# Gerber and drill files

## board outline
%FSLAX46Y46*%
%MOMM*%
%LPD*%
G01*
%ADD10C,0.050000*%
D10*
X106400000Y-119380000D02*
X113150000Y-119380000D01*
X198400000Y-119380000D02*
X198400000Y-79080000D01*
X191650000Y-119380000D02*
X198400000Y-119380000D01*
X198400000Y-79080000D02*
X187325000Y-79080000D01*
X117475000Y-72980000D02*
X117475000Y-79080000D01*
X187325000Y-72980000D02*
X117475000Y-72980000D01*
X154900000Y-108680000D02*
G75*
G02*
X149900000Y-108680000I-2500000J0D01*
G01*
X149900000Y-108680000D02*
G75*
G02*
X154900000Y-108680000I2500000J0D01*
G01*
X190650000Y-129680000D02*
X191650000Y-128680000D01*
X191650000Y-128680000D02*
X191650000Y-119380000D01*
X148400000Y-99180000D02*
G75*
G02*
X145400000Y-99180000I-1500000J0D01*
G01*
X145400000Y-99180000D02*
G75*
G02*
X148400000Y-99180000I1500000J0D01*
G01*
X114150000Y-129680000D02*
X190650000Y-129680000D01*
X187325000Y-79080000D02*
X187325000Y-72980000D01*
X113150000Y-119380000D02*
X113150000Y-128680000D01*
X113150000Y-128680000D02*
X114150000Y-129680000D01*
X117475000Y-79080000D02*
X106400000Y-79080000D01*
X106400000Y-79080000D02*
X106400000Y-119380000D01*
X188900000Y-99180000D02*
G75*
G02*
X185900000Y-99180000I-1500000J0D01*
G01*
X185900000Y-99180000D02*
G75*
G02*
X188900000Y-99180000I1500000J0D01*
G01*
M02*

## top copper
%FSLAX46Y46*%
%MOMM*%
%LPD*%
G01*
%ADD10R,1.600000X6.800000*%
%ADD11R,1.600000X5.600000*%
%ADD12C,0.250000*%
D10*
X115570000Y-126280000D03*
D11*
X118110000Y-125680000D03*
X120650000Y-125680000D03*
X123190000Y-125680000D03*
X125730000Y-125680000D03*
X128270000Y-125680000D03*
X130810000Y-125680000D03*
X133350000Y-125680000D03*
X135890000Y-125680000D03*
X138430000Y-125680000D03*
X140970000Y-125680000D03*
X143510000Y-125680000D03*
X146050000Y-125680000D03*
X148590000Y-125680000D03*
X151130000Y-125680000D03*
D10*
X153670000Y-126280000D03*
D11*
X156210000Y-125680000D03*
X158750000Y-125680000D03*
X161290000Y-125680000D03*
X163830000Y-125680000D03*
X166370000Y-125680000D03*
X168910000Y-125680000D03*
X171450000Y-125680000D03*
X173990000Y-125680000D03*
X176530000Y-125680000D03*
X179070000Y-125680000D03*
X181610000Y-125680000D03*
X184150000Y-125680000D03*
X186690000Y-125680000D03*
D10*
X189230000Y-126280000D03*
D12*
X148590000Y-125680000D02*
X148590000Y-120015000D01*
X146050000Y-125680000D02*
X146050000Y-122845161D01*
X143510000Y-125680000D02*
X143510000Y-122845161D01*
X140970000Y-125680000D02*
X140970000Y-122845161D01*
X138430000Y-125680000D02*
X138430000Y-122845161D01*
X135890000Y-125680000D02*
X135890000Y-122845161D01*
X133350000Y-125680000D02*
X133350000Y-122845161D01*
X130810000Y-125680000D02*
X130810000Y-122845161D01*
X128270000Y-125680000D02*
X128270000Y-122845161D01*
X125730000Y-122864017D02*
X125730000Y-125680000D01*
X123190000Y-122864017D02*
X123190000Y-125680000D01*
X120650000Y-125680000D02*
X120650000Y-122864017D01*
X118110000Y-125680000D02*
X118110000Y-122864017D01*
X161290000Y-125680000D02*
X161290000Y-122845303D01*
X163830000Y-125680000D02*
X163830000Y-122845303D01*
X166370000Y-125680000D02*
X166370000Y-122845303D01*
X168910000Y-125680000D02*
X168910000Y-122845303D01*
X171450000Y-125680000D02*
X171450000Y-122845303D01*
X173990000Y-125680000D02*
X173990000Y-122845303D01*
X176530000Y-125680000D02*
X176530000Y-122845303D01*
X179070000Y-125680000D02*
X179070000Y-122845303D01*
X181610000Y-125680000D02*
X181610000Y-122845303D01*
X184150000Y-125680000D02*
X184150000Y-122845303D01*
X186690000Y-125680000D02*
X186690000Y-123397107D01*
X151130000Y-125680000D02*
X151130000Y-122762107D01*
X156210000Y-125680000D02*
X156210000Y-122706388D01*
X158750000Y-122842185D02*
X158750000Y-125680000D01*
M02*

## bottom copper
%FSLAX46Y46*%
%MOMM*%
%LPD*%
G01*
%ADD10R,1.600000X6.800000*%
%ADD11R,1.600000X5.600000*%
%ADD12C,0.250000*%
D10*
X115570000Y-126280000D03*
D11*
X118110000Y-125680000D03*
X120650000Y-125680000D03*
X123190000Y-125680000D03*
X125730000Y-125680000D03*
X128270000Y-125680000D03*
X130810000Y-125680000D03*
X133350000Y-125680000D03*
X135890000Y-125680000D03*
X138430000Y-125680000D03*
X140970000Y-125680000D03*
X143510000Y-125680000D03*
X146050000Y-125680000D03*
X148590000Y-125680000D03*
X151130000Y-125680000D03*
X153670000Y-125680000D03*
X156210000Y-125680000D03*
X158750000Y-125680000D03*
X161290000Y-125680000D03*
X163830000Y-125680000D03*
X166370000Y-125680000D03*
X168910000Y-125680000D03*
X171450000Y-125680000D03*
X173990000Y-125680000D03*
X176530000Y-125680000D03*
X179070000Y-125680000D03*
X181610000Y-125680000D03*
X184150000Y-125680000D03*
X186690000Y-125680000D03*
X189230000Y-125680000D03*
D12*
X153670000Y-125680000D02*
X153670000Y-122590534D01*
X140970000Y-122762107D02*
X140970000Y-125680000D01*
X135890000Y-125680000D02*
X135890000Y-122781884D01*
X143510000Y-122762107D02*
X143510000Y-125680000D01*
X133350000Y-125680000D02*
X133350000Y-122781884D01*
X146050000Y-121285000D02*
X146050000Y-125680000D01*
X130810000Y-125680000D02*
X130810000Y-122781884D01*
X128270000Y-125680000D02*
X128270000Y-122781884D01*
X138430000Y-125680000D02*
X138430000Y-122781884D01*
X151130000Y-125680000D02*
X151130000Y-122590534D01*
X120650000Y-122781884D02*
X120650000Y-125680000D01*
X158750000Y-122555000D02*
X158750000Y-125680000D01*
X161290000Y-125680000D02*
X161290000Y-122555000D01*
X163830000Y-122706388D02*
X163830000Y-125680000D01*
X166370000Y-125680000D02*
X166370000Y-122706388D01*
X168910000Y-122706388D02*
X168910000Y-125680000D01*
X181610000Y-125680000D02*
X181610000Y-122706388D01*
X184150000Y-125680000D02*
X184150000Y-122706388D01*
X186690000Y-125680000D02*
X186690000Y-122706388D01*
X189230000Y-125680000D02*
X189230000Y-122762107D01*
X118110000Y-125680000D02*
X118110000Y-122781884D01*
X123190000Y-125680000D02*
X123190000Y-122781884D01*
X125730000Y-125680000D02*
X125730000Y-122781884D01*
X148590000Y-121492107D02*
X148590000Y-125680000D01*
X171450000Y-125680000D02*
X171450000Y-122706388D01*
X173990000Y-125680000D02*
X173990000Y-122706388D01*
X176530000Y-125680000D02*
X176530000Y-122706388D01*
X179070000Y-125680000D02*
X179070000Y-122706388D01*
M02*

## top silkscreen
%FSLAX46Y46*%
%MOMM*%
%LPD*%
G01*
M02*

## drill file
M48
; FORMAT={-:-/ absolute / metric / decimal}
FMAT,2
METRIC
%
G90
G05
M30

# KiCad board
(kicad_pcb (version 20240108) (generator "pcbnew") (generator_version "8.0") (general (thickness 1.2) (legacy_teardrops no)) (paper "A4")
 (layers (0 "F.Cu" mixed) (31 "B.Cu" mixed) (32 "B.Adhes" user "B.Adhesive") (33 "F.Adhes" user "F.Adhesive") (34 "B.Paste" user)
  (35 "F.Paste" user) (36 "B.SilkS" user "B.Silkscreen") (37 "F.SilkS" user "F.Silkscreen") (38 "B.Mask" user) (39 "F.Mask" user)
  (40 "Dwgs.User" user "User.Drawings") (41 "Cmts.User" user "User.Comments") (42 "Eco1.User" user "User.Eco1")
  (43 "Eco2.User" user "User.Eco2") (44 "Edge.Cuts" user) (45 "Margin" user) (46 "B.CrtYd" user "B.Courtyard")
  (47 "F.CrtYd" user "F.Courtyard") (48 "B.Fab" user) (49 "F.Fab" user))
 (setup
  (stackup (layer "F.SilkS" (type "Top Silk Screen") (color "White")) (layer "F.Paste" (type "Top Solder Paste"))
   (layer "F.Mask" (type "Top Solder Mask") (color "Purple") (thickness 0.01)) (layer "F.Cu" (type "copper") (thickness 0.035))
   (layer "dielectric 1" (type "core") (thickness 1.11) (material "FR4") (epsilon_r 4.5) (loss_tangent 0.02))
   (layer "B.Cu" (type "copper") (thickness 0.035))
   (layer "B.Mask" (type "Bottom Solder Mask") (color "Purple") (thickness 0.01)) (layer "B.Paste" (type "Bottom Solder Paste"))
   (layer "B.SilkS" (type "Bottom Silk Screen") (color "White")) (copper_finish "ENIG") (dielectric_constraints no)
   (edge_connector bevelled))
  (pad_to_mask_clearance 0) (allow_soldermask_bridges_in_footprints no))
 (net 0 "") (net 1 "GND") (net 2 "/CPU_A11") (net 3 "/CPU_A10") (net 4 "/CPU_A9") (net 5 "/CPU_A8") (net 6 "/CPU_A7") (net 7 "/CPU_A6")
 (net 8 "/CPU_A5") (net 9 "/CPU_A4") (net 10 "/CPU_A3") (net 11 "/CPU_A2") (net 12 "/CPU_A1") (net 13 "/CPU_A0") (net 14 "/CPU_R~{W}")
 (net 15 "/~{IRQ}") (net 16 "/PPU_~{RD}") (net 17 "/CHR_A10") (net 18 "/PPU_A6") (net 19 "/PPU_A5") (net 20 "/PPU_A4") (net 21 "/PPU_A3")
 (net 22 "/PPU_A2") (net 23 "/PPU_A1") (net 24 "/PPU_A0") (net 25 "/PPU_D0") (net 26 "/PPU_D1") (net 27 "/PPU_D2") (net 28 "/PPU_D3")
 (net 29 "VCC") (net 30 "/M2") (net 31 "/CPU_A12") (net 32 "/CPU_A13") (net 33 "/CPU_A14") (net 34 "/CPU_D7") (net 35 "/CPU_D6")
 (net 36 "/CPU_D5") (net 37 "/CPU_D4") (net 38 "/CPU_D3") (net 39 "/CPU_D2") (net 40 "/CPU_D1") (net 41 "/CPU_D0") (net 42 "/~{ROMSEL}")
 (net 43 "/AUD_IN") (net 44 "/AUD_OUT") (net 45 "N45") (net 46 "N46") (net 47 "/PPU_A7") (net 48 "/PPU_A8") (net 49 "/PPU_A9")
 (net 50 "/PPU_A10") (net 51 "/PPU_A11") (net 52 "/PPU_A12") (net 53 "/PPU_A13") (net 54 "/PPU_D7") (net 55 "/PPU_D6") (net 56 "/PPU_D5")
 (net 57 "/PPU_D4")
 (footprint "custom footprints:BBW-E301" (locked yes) (layer "F.Cu") (at 152.4 119.38)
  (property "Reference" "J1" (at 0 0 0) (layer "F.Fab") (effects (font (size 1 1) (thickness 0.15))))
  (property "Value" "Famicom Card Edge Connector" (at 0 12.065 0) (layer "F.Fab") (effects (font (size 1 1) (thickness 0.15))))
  (pad "1" connect rect (at -36.83 6.9) (size 1.6 6.8) (layers "F.Cu") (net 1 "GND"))
  (pad "2" connect rect (at -34.29 6.3) (size 1.6 5.6) (layers "F.Cu") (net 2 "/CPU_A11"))
  (pad "3" connect rect (at -31.75 6.3) (size 1.6 5.6) (layers "F.Cu") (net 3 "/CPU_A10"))
  (pad "4" connect rect (at -29.21 6.3) (size 1.6 5.6) (layers "F.Cu") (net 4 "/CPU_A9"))
  (pad "5" connect rect (at -26.67 6.3) (size 1.6 5.6) (layers "F.Cu") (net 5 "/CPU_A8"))
  (pad "6" connect rect (at -24.13 6.3) (size 1.6 5.6) (layers "F.Cu") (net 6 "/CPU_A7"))
  (pad "7" connect rect (at -21.59 6.3) (size 1.6 5.6) (layers "F.Cu") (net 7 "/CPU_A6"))
  (pad "8" connect rect (at -19.05 6.3) (size 1.6 5.6) (layers "F.Cu") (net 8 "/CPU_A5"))
  (pad "9" connect rect (at -16.51 6.3) (size 1.6 5.6) (layers "F.Cu") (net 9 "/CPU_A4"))
  (pad "10" connect rect (at -13.97 6.3) (size 1.6 5.6) (layers "F.Cu") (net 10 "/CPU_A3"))
  (pad "11" connect rect (at -11.43 6.3) (size 1.6 5.6) (layers "F.Cu") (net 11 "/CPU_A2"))
  (pad "12" connect rect (at -8.89 6.3) (size 1.6 5.6) (layers "F.Cu") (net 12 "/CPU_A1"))
  (pad "13" connect rect (at -6.35 6.3) (size 1.6 5.6) (layers "F.Cu") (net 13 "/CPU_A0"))
  (pad "14" connect rect (at -3.81 6.3) (size 1.6 5.6) (layers "F.Cu") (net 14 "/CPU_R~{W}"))
  (pad "15" connect rect (at -1.27 6.3) (size 1.6 5.6) (layers "F.Cu") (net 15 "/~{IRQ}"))
  (pad "16" connect rect (at 1.27 6.9) (size 1.6 6.8) (layers "F.Cu") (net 1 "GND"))
  (pad "17" connect rect (at 3.81 6.3) (size 1.6 5.6) (layers "F.Cu") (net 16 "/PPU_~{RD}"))
  (pad "18" connect rect (at 6.35 6.3) (size 1.6 5.6) (layers "F.Cu") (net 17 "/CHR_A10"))
  (pad "19" connect rect (at 8.89 6.3) (size 1.6 5.6) (layers "F.Cu") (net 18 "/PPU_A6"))
  (pad "20" connect rect (at 11.43 6.3) (size 1.6 5.6) (layers "F.Cu") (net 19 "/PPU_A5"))
  (pad "21" connect rect (at 13.97 6.3) (size 1.6 5.6) (layers "F.Cu") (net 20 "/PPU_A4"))
  (pad "22" connect rect (at 16.51 6.3) (size 1.6 5.6) (layers "F.Cu") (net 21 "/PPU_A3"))
  (pad "23" connect rect (at 19.05 6.3) (size 1.6 5.6) (layers "F.Cu") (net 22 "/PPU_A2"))
  (pad "24" connect rect (at 21.59 6.3) (size 1.6 5.6) (layers "F.Cu") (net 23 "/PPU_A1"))
  (pad "25" connect rect (at 24.13 6.3) (size 1.6 5.6) (layers "F.Cu") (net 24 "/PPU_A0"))
  (pad "26" connect rect (at 26.67 6.3) (size 1.6 5.6) (layers "F.Cu") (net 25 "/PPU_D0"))
  (pad "27" connect rect (at 29.21 6.3) (size 1.6 5.6) (layers "F.Cu") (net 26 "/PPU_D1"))
  (pad "28" connect rect (at 31.75 6.3) (size 1.6 5.6) (layers "F.Cu") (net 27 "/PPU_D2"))
  (pad "29" connect rect (at 34.29 6.3) (size 1.6 5.6) (layers "F.Cu") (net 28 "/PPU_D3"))
  (pad "30" connect rect (at 36.83 6.9) (size 1.6 6.8) (layers "F.Cu") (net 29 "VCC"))
  (pad "31" connect rect (at -36.83 6.9) (size 1.6 6.8) (layers "B.Cu") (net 29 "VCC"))
  (pad "32" connect rect (at -34.29 6.3) (size 1.6 5.6) (layers "B.Cu") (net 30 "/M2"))
  (pad "33" connect rect (at -31.75 6.3) (size 1.6 5.6) (layers "B.Cu") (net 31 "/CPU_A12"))
  (pad "34" connect rect (at -29.21 6.3) (size 1.6 5.6) (layers "B.Cu") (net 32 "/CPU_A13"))
  (pad "35" connect rect (at -26.67 6.3) (size 1.6 5.6) (layers "B.Cu") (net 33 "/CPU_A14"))
  (pad "36" connect rect (at -24.13 6.3) (size 1.6 5.6) (layers "B.Cu") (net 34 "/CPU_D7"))
  (pad "37" connect rect (at -21.59 6.3) (size 1.6 5.6) (layers "B.Cu") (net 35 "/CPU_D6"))
  (pad "38" connect rect (at -19.05 6.3) (size 1.6 5.6) (layers "B.Cu") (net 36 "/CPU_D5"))
  (pad "39" connect rect (at -16.51 6.3) (size 1.6 5.6) (layers "B.Cu") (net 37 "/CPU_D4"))
  (pad "40" connect rect (at -13.97 6.3) (size 1.6 5.6) (layers "B.Cu") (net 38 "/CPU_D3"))
  (pad "41" connect rect (at -11.43 6.3) (size 1.6 5.6) (layers "B.Cu") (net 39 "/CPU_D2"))
  (pad "42" connect rect (at -8.89 6.3) (size 1.6 5.6) (layers "B.Cu") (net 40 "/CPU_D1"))
  (pad "43" connect rect (at -6.35 6.3) (size 1.6 5.6) (layers "B.Cu") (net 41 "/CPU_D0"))
  (pad "44" connect rect (at -3.81 6.3) (size 1.6 5.6) (layers "B.Cu") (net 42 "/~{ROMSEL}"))
  (pad "45" connect rect (at -1.27 6.3) (size 1.6 5.6) (layers "B.Cu") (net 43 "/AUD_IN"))
  (pad "46" connect rect (at 1.27 6.3) (size 1.6 5.6) (layers "B.Cu") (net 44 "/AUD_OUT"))
  (pad "47" connect rect (at 3.81 6.3) (size 1.6 5.6) (layers "B.Cu") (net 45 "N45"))
  (pad "48" connect rect (at 6.35 6.3) (size 1.6 5.6) (layers "B.Cu") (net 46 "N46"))
  (pad "49" connect rect (at 8.89 6.3) (size 1.6 5.6) (layers "B.Cu") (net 46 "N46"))
  (pad "50" connect rect (at 11.43 6.3) (size 1.6 5.6) (layers "B.Cu") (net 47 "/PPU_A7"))
  (pad "51" connect rect (at 13.97 6.3) (size 1.6 5.6) (layers "B.Cu") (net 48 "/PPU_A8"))
  (pad "52" connect rect (at 16.51 6.3) (size 1.6 5.6) (layers "B.Cu") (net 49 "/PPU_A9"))
  (pad "53" connect rect (at 19.05 6.3) (size 1.6 5.6) (layers "B.Cu") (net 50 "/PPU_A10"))
  (pad "54" connect rect (at 21.59 6.3) (size 1.6 5.6) (layers "B.Cu") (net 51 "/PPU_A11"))
  (pad "55" connect rect (at 24.13 6.3) (size 1.6 5.6) (layers "B.Cu") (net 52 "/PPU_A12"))
  (pad "56" connect rect (at 26.67 6.3) (size 1.6 5.6) (layers "B.Cu") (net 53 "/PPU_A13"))
  (pad "57" connect rect (at 29.21 6.3) (size 1.6 5.6) (layers "B.Cu") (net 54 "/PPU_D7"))
  (pad "58" connect rect (at 31.75 6.3) (size 1.6 5.6) (layers "B.Cu") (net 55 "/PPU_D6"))
  (pad "59" connect rect (at 34.29 6.3) (size 1.6 5.6) (layers "B.Cu") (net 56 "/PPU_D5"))
  (pad "60" connect rect (at 36.83 6.3) (size 1.6 5.6) (layers "B.Cu") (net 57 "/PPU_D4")))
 (gr_line (start 106.4 119.38) (end 113.15 119.38) (stroke (width 0.05) (type solid)) (layer "Edge.Cuts"))
 (gr_line (start 198.4 119.38) (end 198.4 79.08) (stroke (width 0.05) (type solid)) (layer "Edge.Cuts"))
 (gr_line (start 191.65 119.38) (end 198.4 119.38) (stroke (width 0.05) (type solid)) (layer "Edge.Cuts"))
 (gr_line (start 198.4 79.08) (end 187.325 79.08) (stroke (width 0.05) (type solid)) (layer "Edge.Cuts"))
 (gr_line (start 117.475 72.98) (end 117.475 79.08) (stroke (width 0.05) (type solid)) (layer "Edge.Cuts"))
 (gr_line (start 187.325 72.98) (end 117.475 72.98) (stroke (width 0.05) (type solid)) (layer "Edge.Cuts"))
 (gr_circle (center 152.4 108.68) (end 154.9 108.68) (stroke (width 0.05) (type solid)) (fill none) (layer "Edge.Cuts"))
 (gr_line (start 190.65 129.68) (end 191.65 128.68) (stroke (width 0.05) (type solid)) (layer "Edge.Cuts"))
 (gr_line (start 191.65 128.68) (end 191.65 119.38) (stroke (width 0.05) (type solid)) (layer "Edge.Cuts"))
 (gr_circle (center 146.9 99.18) (end 148.4 99.18) (stroke (width 0.05) (type solid)) (fill none) (layer "Edge.Cuts"))
 (gr_line (start 114.15 129.68) (end 190.65 129.68) (stroke (width 0.05) (type solid)) (layer "Edge.Cuts"))
 (gr_line (start 187.325 79.08) (end 187.325 72.98) (stroke (width 0.05) (type solid)) (layer "Edge.Cuts"))
 (gr_line (start 113.15 119.38) (end 113.15 128.68) (stroke (width 0.05) (type solid)) (layer "Edge.Cuts"))
 (gr_line (start 113.15 128.68) (end 114.15 129.68) (stroke (width 0.05) (type solid)) (layer "Edge.Cuts"))
 (gr_line (start 117.475 79.08) (end 106.4 79.08) (stroke (width 0.05) (type solid)) (layer "Edge.Cuts"))
 (gr_line (start 106.4 79.08) (end 106.4 119.38) (stroke (width 0.05) (type solid)) (layer "Edge.Cuts"))
 (gr_circle (center 187.4 99.18) (end 188.9 99.18) (stroke (width 0.05) (type solid)) (fill none) (layer "Edge.Cuts"))
 (segment (start 153.67 125.68) (end 153.67 122.590534) (width 0.25) (layer "B.Cu") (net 44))
 (segment (start 140.97 122.762107) (end 140.97 125.68) (width 0.25) (layer "B.Cu") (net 39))
 (segment (start 135.89 125.68) (end 135.89 122.781884) (width 0.25) (layer "B.Cu") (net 37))
 (segment (start 143.51 122.762107) (end 143.51 125.68) (width 0.25) (layer "B.Cu") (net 40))
 (segment (start 133.35 125.68) (end 133.35 122.781884) (width 0.25) (layer "B.Cu") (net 36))
 (segment (start 146.05 121.285) (end 146.05 125.68) (width 0.25) (layer "B.Cu") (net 41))
 (segment (start 130.81 125.68) (end 130.81 122.781884) (width 0.25) (layer "B.Cu") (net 35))
 (segment (start 128.27 125.68) (end 128.27 122.781884) (width 0.25) (layer "B.Cu") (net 34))
 (segment (start 148.59 125.68) (end 148.59 120.015) (width 0.25) (layer "F.Cu") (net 14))
 (segment (start 138.43 125.68) (end 138.43 122.781884) (width 0.25) (layer "B.Cu") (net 38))
 (segment (start 151.13 125.68) (end 151.13 122.590534) (width 0.25) (layer "B.Cu") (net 43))
 (segment (start 120.65 122.781884) (end 120.65 125.68) (width 0.25) (layer "B.Cu") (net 31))
 (segment (start 146.05 125.68) (end 146.05 122.845161) (width 0.25) (layer "F.Cu") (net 13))
 (segment (start 143.51 125.68) (end 143.51 122.845161) (width 0.25) (layer "F.Cu") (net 12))
 (segment (start 140.97 125.68) (end 140.97 122.845161) (width 0.25) (layer "F.Cu") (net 11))
 (segment (start 138.43 125.68) (end 138.43 122.845161) (width 0.25) (layer "F.Cu") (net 10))
 (segment (start 135.89 125.68) (end 135.89 122.845161) (width 0.25) (layer "F.Cu") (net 9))
 (segment (start 133.35 125.68) (end 133.35 122.845161) (width 0.25) (layer "F.Cu") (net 8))
 (segment (start 130.81 125.68) (end 130.81 122.845161) (width 0.25) (layer "F.Cu") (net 7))
 (segment (start 128.27 125.68) (end 128.27 122.845161) (width 0.25) (layer "F.Cu") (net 6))
 (segment (start 125.73 122.864017) (end 125.73 125.68) (width 0.25) (layer "F.Cu") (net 5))
 (segment (start 123.19 122.864017) (end 123.19 125.68) (width 0.25) (layer "F.Cu") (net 4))
 (segment (start 120.65 125.68) (end 120.65 122.864017) (width 0.25) (layer "F.Cu") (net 3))
 (segment (start 118.11 125.68) (end 118.11 122.864017) (width 0.25) (layer "F.Cu") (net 2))
 (segment (start 158.75 122.555) (end 158.75 125.68) (width 0.25) (layer "B.Cu") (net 46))
 (segment (start 161.29 125.68) (end 161.29 122.555) (width 0.25) (layer "B.Cu") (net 46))
 (segment (start 161.29 125.68) (end 161.29 122.845303) (width 0.25) (layer "F.Cu") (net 18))
 (segment (start 163.83 125.68) (end 163.83 122.845303) (width 0.25) (layer "F.Cu") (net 19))
 (segment (start 166.37 125.68) (end 166.37 122.845303) (width 0.25) (layer "F.Cu") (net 20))
 (segment (start 168.91 125.68) (end 168.91 122.845303) (width 0.25) (layer "F.Cu") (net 21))
 (segment (start 171.45 125.68) (end 171.45 122.845303) (width 0.25) (layer "F.Cu") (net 22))
 (segment (start 173.99 125.68) (end 173.99 122.845303) (width 0.25) (layer "F.Cu") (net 23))
 (segment (start 176.53 125.68) (end 176.53 122.845303) (width 0.25) (layer "F.Cu") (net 24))
 (segment (start 179.07 125.68) (end 179.07 122.845303) (width 0.25) (layer "F.Cu") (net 25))
 (segment (start 181.61 125.68) (end 181.61 122.845303) (width 0.25) (layer "F.Cu") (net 26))
 (segment (start 184.15 125.68) (end 184.15 122.845303) (width 0.25) (layer "F.Cu") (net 27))
 (segment (start 186.69 125.68) (end 186.69 123.397107) (width 0.25) (layer "F.Cu") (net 28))
 (segment (start 163.83 122.706388) (end 163.83 125.68) (width 0.25) (layer "B.Cu") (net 47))
 (segment (start 166.37 125.68) (end 166.37 122.706388) (width 0.25) (layer "B.Cu") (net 48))
 (segment (start 168.91 122.706388) (end 168.91 125.68) (width 0.25) (layer "B.Cu") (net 49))
 (segment (start 181.61 125.68) (end 181.61 122.706388) (width 0.25) (layer "B.Cu") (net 54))
 (segment (start 184.15 125.68) (end 184.15 122.706388) (width 0.25) (layer "B.Cu") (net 55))
 (segment (start 186.69 125.68) (end 186.69 122.706388) (width 0.25) (layer "B.Cu") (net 56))
 (segment (start 189.23 125.68) (end 189.23 122.762107) (width 0.25) (layer "B.Cu") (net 57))
 (segment (start 118.11 125.68) (end 118.11 122.781884) (width 0.25) (layer "B.Cu") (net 30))
 (segment (start 123.19 125.68) (end 123.19 122.781884) (width 0.25) (layer "B.Cu") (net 32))
 (segment (start 125.73 125.68) (end 125.73 122.781884) (width 0.25) (layer "B.Cu") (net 33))
 (segment (start 148.59 121.492107) (end 148.59 125.68) (width 0.25) (layer "B.Cu") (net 42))
 (segment (start 151.13 125.68) (end 151.13 122.762107) (width 0.25) (layer "F.Cu") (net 15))
 (segment (start 156.21 125.68) (end 156.21 122.706388) (width 0.25) (layer "F.Cu") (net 16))
 (segment (start 171.45 125.68) (end 171.45 122.706388) (width 0.25) (layer "B.Cu") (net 50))
 (segment (start 173.99 125.68) (end 173.99 122.706388) (width 0.25) (layer "B.Cu") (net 51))
 (segment (start 176.53 125.68) (end 176.53 122.706388) (width 0.25) (layer "B.Cu") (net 52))
 (segment (start 179.07 125.68) (end 179.07 122.706388) (width 0.25) (layer "B.Cu") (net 53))
 (segment (start 158.75 122.842185) (end 158.75 125.68) (width 0.25) (layer "F.Cu") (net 17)))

